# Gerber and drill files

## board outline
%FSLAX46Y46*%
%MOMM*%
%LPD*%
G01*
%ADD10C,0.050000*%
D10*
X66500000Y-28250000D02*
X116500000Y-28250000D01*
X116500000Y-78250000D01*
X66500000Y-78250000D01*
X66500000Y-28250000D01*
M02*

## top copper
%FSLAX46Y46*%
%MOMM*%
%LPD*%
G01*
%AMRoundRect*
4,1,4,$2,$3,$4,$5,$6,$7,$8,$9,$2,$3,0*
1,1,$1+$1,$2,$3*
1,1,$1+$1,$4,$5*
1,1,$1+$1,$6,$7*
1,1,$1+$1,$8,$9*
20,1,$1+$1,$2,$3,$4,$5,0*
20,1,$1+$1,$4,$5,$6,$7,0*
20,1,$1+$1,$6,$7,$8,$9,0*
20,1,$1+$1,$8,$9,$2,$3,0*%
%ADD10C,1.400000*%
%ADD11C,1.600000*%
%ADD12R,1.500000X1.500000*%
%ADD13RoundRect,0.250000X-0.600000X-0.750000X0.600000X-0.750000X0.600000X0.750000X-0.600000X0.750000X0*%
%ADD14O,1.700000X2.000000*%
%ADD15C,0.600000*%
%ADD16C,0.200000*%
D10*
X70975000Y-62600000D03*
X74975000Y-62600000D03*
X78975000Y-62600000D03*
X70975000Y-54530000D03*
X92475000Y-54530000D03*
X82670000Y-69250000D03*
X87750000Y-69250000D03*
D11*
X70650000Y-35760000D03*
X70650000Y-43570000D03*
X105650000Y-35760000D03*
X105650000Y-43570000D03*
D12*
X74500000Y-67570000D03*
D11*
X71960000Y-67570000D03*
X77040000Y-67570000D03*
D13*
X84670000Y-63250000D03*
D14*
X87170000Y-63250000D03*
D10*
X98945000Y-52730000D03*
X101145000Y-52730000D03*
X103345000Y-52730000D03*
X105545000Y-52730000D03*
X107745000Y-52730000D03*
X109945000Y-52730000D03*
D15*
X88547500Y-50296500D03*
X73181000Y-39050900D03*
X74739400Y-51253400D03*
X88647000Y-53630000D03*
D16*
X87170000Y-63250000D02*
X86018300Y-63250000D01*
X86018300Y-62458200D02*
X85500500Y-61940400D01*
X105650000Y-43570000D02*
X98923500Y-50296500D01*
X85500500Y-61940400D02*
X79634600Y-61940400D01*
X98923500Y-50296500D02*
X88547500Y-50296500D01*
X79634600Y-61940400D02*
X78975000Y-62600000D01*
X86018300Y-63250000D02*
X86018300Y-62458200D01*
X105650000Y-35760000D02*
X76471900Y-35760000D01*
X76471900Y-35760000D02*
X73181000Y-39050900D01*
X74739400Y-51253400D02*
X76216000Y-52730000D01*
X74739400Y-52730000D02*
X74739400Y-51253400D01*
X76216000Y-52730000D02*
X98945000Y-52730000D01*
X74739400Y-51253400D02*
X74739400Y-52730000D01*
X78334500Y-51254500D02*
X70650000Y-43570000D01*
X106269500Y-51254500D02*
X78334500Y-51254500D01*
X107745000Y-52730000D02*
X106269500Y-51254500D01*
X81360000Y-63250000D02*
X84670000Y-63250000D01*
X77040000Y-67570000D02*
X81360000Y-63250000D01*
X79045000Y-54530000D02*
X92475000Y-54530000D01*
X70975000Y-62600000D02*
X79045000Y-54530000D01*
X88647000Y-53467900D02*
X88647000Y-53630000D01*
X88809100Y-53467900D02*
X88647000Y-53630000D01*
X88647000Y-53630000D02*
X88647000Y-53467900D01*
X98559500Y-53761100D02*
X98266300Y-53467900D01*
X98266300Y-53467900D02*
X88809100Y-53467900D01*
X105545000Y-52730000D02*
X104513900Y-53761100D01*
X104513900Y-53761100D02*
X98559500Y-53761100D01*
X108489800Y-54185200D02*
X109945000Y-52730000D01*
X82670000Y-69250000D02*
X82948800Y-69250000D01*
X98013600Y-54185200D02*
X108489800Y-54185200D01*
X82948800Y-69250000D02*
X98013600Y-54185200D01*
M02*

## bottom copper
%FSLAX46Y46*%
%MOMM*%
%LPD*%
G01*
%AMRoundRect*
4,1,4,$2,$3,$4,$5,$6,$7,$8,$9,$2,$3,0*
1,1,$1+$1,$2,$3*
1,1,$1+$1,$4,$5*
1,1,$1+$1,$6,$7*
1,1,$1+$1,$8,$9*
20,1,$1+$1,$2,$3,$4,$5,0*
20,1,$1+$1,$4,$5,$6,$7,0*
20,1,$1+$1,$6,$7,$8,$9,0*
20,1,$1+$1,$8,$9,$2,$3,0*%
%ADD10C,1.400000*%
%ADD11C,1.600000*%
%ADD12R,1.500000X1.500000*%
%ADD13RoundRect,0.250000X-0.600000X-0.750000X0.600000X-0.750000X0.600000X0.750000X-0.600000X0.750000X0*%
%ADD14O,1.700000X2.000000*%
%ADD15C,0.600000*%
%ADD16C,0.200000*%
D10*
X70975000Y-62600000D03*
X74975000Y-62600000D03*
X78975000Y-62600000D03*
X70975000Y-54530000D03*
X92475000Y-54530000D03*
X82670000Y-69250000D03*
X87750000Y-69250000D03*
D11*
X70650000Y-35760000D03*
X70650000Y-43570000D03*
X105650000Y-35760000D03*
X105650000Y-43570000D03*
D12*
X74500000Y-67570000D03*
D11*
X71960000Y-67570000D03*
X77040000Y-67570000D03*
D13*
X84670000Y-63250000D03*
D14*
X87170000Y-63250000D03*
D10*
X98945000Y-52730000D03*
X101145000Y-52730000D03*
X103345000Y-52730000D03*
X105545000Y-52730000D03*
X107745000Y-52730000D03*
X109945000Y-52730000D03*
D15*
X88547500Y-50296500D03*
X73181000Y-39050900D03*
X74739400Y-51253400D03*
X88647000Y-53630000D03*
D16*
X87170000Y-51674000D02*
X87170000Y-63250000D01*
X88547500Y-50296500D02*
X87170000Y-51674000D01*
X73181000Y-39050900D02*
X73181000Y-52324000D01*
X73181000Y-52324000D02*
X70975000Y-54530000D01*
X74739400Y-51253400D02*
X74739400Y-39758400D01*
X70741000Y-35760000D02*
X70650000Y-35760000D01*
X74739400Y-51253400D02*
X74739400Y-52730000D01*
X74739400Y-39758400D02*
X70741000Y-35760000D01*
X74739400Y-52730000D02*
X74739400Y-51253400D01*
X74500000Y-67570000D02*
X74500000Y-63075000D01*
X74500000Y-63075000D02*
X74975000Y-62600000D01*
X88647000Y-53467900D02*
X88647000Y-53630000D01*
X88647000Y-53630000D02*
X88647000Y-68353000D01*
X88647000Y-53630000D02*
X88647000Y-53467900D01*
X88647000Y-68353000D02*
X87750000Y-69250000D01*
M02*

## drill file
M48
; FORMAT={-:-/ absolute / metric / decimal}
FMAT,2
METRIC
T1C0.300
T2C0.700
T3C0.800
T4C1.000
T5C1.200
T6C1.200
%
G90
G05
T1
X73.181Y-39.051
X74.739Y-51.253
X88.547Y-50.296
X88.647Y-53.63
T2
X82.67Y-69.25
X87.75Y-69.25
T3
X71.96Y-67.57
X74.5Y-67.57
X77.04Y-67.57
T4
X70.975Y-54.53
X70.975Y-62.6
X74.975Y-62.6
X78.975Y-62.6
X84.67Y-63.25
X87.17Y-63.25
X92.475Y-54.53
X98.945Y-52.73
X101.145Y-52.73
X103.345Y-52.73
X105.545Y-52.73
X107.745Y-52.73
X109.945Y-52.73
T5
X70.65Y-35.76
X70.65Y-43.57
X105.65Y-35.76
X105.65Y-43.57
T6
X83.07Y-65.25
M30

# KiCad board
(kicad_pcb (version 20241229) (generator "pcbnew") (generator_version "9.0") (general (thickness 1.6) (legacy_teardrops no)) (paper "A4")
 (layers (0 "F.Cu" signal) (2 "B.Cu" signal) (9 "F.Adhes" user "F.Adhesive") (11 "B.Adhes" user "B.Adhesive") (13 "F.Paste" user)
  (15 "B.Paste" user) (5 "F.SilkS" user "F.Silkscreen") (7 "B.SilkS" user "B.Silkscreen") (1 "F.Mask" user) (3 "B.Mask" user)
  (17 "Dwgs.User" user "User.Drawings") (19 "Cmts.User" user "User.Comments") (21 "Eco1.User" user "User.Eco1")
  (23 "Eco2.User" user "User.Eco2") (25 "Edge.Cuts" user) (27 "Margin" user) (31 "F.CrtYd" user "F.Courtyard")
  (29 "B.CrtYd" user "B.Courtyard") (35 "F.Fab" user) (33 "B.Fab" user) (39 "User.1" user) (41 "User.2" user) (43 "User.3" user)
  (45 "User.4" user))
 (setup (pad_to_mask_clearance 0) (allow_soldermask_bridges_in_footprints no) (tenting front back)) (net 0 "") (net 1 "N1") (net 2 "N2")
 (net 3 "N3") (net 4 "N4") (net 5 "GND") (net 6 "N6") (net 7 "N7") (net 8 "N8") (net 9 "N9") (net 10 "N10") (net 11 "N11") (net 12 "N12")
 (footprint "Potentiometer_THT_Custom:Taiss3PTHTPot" (layer "F.Cu") (at 69.475 64.8)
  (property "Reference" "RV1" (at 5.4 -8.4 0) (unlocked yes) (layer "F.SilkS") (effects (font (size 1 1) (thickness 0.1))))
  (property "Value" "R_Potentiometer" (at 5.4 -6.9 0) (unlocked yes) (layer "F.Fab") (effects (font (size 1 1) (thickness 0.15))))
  (pad "1" thru_hole circle (at 1.5 -2.2) (size 1.4 1.4) (drill 1) (layers "*.Cu" "*.Mask") (remove_unused_layers no) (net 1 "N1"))
  (pad "2" thru_hole circle (at 5.5 -2.2 90) (size 1.4 1.4) (drill 1) (layers "*.Cu" "*.Mask") (remove_unused_layers no) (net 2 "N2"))
  (pad "3" thru_hole circle (at 9.5 -2.2) (size 1.4 1.4) (drill 1) (layers "*.Cu" "*.Mask") (remove_unused_layers no) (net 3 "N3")))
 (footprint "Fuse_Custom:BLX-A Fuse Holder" (layer "F.Cu") (at 69.475 59.13)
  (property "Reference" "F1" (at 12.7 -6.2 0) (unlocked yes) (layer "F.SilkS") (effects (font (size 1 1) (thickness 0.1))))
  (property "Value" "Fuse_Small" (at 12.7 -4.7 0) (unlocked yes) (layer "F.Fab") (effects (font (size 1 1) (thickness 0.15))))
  (pad "1" thru_hole circle (at 1.5 -4.6) (size 1.4 1.4) (drill 1) (layers "*.Cu" "*.Mask") (remove_unused_layers no) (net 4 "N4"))
  (pad "2" thru_hole circle (at 23 -4.6) (size 1.4 1.4) (drill 1) (layers "*.Cu" "*.Mask") (remove_unused_layers no) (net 1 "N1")))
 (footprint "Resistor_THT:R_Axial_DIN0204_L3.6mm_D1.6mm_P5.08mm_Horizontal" (layer "F.Cu") (at 82.67 69.25)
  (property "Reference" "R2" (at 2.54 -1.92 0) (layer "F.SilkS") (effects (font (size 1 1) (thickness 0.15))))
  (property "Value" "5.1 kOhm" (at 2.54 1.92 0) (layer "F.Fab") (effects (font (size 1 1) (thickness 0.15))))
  (pad "1" thru_hole circle (at 0 0) (size 1.4 1.4) (drill 0.7) (layers "*.Cu" "*.Mask") (remove_unused_layers no) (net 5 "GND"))
  (pad "2" thru_hole circle (at 5.08 0) (size 1.4 1.4) (drill 0.7) (layers "*.Cu" "*.Mask") (remove_unused_layers no) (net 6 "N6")))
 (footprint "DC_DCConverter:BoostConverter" (layer "F.Cu") (at 69.65 48.26)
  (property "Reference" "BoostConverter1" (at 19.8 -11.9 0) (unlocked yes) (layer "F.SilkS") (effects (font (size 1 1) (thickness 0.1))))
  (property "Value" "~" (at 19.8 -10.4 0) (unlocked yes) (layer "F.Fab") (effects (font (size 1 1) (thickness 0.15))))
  (pad "1" thru_hole circle (at 1 -12.5) (size 1.6 1.6) (drill 1.2) (layers "*.Cu" "*.Mask") (remove_unused_layers no) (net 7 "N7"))
  (pad "2" thru_hole circle (at 1 -4.69) (size 1.6 1.6) (drill 1.2) (layers "*.Cu" "*.Mask") (remove_unused_layers no) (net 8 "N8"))
  (pad "3" thru_hole circle (at 36 -12.5) (size 1.6 1.6) (drill 1.2) (layers "*.Cu" "*.Mask") (remove_unused_layers no) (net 4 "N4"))
  (pad "4" thru_hole circle (at 36 -4.69) (size 1.6 1.6) (drill 1.2) (layers "*.Cu" "*.Mask") (remove_unused_layers no) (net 3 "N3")))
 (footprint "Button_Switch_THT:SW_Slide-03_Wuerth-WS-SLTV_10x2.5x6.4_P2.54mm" (layer "F.Cu") (at 74.5 67.57)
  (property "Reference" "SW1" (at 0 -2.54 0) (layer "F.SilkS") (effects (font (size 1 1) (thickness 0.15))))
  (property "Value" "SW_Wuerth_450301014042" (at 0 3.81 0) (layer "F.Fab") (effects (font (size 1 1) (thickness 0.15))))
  (pad "1" thru_hole rect (at 0 0) (size 1.5 1.5) (drill 0.8) (layers "*.Cu" "*.Mask") (remove_unused_layers no) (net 2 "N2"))
  (pad "2" thru_hole circle (at -2.54 0) (size 1.6 1.6) (drill 0.8) (layers "*.Cu" "*.Mask") (remove_unused_layers no) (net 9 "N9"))
  (pad "3" thru_hole circle (at 2.54 0) (size 1.6 1.6) (drill 0.8) (layers "*.Cu" "*.Mask") (remove_unused_layers no) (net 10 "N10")))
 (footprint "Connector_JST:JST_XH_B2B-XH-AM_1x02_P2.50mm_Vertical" (layer "F.Cu") (at 84.67 63.25)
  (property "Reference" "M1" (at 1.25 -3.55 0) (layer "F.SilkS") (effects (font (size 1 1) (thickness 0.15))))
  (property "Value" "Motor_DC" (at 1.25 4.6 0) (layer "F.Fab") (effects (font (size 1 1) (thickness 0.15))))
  (pad "" np_thru_hole circle (at -1.6 2) (size 1.2 1.2) (drill 1.2) (layers "*.Cu" "*.Mask"))
  (pad "1" thru_hole roundrect (at 0 0) (size 1.7 2) (drill 1) (layers "*.Cu" "*.Mask") (remove_unused_layers no)
   (roundrect_rratio 0.147059) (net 10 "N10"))
  (pad "2" thru_hole oval (at 2.5 0) (size 1.7 2) (drill 1) (layers "*.Cu" "*.Mask") (remove_unused_layers no) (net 3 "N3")))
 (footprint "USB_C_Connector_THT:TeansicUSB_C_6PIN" (layer "F.Cu") (at 96.345 64.73)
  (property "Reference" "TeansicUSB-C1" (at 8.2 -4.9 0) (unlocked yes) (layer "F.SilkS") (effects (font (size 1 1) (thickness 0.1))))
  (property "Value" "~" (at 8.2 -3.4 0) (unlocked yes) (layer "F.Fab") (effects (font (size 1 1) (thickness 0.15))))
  (pad "1" thru_hole circle (at 2.6 -12) (size 1.4 1.4) (drill 1) (layers "*.Cu" "*.Mask") (remove_unused_layers no) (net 7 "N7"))
  (pad "2" thru_hole circle (at 4.8 -12) (size 1.4 1.4) (drill 1) (layers "*.Cu" "*.Mask") (remove_unused_layers no) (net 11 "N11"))
  (pad "3" thru_hole circle (at 7 -12) (size 1.4 1.4) (drill 1) (layers "*.Cu" "*.Mask") (remove_unused_layers no) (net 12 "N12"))
  (pad "4" thru_hole circle (at 9.2 -12) (size 1.4 1.4) (drill 1) (layers "*.Cu" "*.Mask") (remove_unused_layers no) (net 6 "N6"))
  (pad "5" thru_hole circle (at 11.4 -12) (size 1.4 1.4) (drill 1) (layers "*.Cu" "*.Mask") (remove_unused_layers no) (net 8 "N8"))
  (pad "6" thru_hole circle (at 13.6 -12) (size 1.4 1.4) (drill 1) (layers "*.Cu" "*.Mask") (remove_unused_layers no) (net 5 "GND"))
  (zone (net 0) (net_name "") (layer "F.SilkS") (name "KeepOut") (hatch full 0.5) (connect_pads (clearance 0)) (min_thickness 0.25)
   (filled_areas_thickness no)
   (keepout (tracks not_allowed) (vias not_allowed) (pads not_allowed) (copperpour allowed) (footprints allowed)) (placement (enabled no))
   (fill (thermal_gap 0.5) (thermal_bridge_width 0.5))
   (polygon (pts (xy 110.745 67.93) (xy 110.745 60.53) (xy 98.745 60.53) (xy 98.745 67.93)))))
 (gr_rect (start 66.5 28.25) (end 116.5 78.25) (stroke (width 0.05) (type default)) (fill no) (layer "Edge.Cuts"))
 (segment (start 87.17 63.25) (end 86.0183 63.25) (width 0.2) (layer "F.Cu") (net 3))
 (segment (start 86.0183 62.4582) (end 85.5005 61.9404) (width 0.2) (layer "F.Cu") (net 3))
 (segment (start 105.65 43.57) (end 98.9235 50.2965) (width 0.2) (layer "F.Cu") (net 3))
 (segment (start 85.5005 61.9404) (end 79.6346 61.9404) (width 0.2) (layer "F.Cu") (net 3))
 (segment (start 98.9235 50.2965) (end 88.5475 50.2965) (width 0.2) (layer "F.Cu") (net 3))
 (segment (start 79.6346 61.9404) (end 78.975 62.6) (width 0.2) (layer "F.Cu") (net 3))
 (segment (start 86.0183 63.25) (end 86.0183 62.4582) (width 0.2) (layer "F.Cu") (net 3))
 (via (at 88.5475 50.2965) (size 0.6) (drill 0.3) (layers "F.Cu" "B.Cu") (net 3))
 (segment (start 87.17 51.674) (end 87.17 63.25) (width 0.2) (layer "B.Cu") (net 3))
 (segment (start 88.5475 50.2965) (end 87.17 51.674) (width 0.2) (layer "B.Cu") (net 3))
 (segment (start 105.65 35.76) (end 76.4719 35.76) (width 0.2) (layer "F.Cu") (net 4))
 (segment (start 76.4719 35.76) (end 73.181 39.0509) (width 0.2) (layer "F.Cu") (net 4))
 (via (at 73.181 39.0509) (size 0.6) (drill 0.3) (layers "F.Cu" "B.Cu") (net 4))
 (segment (start 73.181 39.0509) (end 73.181 52.324) (width 0.2) (layer "B.Cu") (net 4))
 (segment (start 73.181 52.324) (end 70.975 54.53) (width 0.2) (layer "B.Cu") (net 4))
 (segment (start 74.7394 51.2534) (end 76.216 52.73) (width 0.2) (layer "F.Cu") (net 7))
 (segment (start 74.7394 52.73) (end 74.7394 51.2534) (width 0.2) (layer "F.Cu") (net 7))
 (segment (start 76.216 52.73) (end 98.945 52.73) (width 0.2) (layer "F.Cu") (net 7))
 (segment (start 74.7394 51.2534) (end 74.7394 52.73) (width 0.2) (layer "F.Cu") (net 7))
 (via (at 74.7394 51.2534) (size 0.6) (drill 0.3) (layers "F.Cu" "B.Cu") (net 7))
 (segment (start 74.7394 51.2534) (end 74.7394 39.7584) (width 0.2) (layer "B.Cu") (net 7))
 (segment (start 70.741 35.76) (end 70.65 35.76) (width 0.2) (layer "B.Cu") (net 7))
 (segment (start 74.7394 51.2534) (end 74.7394 52.73) (width 0.2) (layer "B.Cu") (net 7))
 (segment (start 74.7394 39.7584) (end 70.741 35.76) (width 0.2) (layer "B.Cu") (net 7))
 (segment (start 74.7394 52.73) (end 74.7394 51.2534) (width 0.2) (layer "B.Cu") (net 7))
 (segment (start 78.3345 51.2545) (end 70.65 43.57) (width 0.2) (layer "F.Cu") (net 8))
 (segment (start 106.2695 51.2545) (end 78.3345 51.2545) (width 0.2) (layer "F.Cu") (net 8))
 (segment (start 107.745 52.73) (end 106.2695 51.2545) (width 0.2) (layer "F.Cu") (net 8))
 (segment (start 74.5 67.57) (end 74.5 63.075) (width 0.2) (layer "B.Cu") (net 2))
 (segment (start 74.5 63.075) (end 74.975 62.6) (width 0.2) (layer "B.Cu") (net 2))
 (segment (start 81.36 63.25) (end 84.67 63.25) (width 0.2) (layer "F.Cu") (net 10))
 (segment (start 77.04 67.57) (end 81.36 63.25) (width 0.2) (layer "F.Cu") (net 10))
 (segment (start 79.045 54.53) (end 92.475 54.53) (width 0.2) (layer "F.Cu") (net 1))
 (segment (start 70.975 62.6) (end 79.045 54.53) (width 0.2) (layer "F.Cu") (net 1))
 (segment (start 88.647 53.4679) (end 88.647 53.63) (width 0.2) (layer "F.Cu") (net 6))
 (segment (start 88.8091 53.4679) (end 88.647 53.63) (width 0.2) (layer "F.Cu") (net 6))
 (segment (start 88.647 53.63) (end 88.647 53.4679) (width 0.2) (layer "F.Cu") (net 6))
 (segment (start 98.5595 53.7611) (end 98.2663 53.4679) (width 0.2) (layer "F.Cu") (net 6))
 (segment (start 98.2663 53.4679) (end 88.8091 53.4679) (width 0.2) (layer "F.Cu") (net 6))
 (segment (start 105.545 52.73) (end 104.5139 53.7611) (width 0.2) (layer "F.Cu") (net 6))
 (segment (start 104.5139 53.7611) (end 98.5595 53.7611) (width 0.2) (layer "F.Cu") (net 6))
 (via (at 88.647 53.63) (size 0.6) (drill 0.3) (layers "F.Cu" "B.Cu") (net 6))
 (segment (start 88.647 53.4679) (end 88.647 53.63) (width 0.2) (layer "B.Cu") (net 6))
 (segment (start 88.647 53.63) (end 88.647 68.353) (width 0.2) (layer "B.Cu") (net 6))
 (segment (start 88.647 53.63) (end 88.647 53.4679) (width 0.2) (layer "B.Cu") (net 6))
 (segment (start 88.647 68.353) (end 87.75 69.25) (width 0.2) (layer "B.Cu") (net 6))
 (segment (start 108.4898 54.1852) (end 109.945 52.73) (width 0.2) (layer "F.Cu") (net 5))
 (segment (start 82.67 69.25) (end 82.9488 69.25) (width 0.2) (layer "F.Cu") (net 5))
 (segment (start 98.0136 54.1852) (end 108.4898 54.1852) (width 0.2) (layer "F.Cu") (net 5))
 (segment (start 82.9488 69.25) (end 98.0136 54.1852) (width 0.2) (layer "F.Cu") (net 5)))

